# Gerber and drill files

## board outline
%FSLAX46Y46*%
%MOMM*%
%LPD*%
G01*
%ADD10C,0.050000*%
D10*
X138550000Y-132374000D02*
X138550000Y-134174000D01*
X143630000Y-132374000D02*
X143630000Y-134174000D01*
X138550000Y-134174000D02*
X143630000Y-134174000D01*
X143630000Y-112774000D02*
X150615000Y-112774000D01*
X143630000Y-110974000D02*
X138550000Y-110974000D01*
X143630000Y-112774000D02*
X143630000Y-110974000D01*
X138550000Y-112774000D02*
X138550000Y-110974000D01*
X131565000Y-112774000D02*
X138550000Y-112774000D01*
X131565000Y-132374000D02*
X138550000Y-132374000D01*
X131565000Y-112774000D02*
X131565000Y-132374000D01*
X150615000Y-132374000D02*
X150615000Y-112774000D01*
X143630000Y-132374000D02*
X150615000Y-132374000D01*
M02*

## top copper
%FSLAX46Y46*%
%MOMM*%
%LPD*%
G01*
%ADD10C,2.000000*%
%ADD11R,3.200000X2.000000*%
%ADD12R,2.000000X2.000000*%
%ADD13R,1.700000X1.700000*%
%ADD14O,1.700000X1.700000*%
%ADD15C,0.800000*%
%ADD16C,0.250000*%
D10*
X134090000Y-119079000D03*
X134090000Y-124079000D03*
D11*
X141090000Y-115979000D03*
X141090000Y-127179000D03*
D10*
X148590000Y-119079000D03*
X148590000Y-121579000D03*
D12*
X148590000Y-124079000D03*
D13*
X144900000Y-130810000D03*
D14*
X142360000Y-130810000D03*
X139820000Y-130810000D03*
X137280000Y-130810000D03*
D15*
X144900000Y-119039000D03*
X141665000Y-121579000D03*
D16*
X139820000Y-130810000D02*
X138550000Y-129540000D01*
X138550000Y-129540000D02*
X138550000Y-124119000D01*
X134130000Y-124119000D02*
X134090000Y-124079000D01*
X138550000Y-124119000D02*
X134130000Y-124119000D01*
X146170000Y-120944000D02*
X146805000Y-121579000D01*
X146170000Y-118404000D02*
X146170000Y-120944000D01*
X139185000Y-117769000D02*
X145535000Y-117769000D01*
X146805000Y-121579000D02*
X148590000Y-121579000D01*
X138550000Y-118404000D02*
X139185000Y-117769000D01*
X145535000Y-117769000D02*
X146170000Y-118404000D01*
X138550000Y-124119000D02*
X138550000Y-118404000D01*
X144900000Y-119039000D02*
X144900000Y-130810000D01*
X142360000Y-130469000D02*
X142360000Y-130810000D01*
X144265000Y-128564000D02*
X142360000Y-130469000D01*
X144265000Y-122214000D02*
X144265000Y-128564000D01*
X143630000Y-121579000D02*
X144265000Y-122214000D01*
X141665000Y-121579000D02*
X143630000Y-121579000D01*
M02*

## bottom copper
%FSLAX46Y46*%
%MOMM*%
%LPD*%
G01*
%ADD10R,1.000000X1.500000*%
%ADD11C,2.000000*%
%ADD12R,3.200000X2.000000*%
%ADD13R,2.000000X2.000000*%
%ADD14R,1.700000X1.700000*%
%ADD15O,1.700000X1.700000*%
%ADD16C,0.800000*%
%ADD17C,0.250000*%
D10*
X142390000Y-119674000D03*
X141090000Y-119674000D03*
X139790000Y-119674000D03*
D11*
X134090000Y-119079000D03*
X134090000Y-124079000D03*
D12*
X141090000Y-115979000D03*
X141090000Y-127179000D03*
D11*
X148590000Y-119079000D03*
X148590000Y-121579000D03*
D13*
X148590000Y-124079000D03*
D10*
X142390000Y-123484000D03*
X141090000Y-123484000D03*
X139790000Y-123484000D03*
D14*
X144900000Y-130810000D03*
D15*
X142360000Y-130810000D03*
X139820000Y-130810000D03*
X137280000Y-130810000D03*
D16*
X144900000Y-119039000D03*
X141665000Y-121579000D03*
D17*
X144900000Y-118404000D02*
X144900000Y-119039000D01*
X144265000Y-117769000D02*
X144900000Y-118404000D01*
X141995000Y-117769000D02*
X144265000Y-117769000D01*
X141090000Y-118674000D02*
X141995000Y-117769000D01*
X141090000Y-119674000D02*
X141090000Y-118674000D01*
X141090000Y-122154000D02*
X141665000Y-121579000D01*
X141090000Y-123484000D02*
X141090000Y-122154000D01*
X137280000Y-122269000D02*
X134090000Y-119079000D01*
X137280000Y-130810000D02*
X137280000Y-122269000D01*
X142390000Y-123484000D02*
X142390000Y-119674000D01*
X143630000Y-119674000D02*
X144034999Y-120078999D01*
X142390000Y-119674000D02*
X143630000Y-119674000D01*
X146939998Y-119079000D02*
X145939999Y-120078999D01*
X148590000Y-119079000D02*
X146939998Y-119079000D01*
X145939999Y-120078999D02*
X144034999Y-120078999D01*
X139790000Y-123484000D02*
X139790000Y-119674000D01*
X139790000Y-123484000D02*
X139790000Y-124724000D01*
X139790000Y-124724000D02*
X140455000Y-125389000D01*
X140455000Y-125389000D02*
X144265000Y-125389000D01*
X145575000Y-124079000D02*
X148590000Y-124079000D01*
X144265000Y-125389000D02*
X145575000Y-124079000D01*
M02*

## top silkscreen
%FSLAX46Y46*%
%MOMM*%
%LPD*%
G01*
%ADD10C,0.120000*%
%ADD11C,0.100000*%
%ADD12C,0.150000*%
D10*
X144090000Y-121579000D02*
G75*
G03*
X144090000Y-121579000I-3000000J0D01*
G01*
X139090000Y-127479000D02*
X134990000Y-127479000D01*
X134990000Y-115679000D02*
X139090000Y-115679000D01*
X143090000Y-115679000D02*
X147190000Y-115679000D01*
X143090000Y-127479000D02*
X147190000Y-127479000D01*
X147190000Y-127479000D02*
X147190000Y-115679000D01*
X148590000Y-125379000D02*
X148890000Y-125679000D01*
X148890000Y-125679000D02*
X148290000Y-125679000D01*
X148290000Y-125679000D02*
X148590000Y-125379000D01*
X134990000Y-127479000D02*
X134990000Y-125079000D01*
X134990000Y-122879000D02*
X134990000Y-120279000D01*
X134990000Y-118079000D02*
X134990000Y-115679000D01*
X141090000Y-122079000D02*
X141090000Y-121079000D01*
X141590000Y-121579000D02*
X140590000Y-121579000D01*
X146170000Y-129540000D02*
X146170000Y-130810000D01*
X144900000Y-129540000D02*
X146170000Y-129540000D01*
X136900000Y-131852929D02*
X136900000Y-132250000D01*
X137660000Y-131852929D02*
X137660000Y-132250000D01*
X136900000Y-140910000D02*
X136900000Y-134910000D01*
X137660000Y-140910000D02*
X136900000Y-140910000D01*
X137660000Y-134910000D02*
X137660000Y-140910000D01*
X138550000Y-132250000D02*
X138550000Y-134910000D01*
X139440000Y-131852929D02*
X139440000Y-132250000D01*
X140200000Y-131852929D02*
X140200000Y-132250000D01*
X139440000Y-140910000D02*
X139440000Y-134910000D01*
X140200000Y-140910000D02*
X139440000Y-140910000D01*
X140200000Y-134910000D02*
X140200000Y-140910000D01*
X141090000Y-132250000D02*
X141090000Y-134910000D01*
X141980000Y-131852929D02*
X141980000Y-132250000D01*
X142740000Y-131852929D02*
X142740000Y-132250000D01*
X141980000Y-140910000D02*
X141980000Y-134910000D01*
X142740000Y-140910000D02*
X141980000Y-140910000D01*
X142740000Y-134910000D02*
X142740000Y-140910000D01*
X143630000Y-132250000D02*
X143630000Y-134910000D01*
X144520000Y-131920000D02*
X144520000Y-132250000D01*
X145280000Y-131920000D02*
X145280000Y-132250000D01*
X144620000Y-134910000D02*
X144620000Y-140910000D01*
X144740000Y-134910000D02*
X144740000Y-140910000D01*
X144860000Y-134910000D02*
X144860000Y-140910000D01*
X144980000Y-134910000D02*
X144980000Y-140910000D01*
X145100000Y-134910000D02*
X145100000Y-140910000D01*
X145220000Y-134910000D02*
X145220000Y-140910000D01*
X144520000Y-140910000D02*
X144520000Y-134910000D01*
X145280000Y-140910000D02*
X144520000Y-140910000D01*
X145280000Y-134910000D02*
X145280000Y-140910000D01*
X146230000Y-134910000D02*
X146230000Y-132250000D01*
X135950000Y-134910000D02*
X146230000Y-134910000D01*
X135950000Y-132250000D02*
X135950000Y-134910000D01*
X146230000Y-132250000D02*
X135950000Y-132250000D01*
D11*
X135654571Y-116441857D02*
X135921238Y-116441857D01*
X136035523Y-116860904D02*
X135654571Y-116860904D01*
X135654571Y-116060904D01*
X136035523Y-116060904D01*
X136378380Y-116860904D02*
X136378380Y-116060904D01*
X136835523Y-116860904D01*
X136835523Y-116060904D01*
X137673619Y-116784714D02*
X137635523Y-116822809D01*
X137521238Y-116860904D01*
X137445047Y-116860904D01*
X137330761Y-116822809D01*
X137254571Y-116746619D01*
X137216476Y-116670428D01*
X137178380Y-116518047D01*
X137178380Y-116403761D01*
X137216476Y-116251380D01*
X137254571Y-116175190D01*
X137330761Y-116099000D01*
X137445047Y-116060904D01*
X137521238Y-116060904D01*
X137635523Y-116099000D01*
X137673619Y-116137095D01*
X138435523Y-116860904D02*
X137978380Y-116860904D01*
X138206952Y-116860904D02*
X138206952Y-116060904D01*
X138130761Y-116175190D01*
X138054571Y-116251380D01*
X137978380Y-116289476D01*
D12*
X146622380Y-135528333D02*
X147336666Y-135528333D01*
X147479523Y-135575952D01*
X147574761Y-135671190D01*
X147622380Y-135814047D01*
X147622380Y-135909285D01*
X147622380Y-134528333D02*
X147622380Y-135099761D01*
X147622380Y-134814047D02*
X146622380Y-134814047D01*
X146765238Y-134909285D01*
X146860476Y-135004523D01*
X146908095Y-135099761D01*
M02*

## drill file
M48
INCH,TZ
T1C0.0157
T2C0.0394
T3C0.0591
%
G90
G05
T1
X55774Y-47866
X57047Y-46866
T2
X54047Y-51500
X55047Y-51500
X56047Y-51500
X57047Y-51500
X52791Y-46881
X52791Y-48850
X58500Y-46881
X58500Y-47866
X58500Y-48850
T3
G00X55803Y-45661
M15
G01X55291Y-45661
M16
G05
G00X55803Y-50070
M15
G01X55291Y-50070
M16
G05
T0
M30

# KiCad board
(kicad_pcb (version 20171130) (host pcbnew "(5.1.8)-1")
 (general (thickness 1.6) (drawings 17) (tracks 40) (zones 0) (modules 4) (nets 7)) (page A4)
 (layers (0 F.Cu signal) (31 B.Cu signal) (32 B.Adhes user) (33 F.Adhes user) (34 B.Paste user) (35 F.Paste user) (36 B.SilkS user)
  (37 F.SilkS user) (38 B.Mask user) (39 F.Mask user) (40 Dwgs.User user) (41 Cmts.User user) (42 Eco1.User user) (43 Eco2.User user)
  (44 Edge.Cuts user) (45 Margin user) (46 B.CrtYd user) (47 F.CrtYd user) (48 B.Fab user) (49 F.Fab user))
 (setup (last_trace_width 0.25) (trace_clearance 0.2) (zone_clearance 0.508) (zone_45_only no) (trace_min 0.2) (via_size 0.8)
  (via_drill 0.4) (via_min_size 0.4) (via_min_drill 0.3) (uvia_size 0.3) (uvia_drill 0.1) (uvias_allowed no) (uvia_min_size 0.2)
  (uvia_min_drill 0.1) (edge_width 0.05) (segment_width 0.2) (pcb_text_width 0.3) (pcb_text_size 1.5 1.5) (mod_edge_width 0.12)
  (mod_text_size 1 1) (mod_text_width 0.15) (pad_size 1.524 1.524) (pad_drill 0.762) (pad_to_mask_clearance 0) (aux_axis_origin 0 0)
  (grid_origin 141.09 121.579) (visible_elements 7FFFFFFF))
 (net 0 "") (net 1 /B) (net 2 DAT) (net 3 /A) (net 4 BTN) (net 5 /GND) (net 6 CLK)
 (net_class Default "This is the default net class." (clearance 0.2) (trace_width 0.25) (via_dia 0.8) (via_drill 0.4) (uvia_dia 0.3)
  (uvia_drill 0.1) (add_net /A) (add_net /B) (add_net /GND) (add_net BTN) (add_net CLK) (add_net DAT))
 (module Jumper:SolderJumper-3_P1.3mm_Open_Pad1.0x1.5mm (layer B.Cu) (at 141.09 119.674 180)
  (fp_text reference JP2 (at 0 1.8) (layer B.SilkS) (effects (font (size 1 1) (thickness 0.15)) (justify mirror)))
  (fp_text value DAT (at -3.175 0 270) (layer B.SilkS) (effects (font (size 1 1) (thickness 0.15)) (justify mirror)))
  (pad 1 smd rect (at -1.3 0 180) (size 1 1.5) (layers B.Cu B.Mask) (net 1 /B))
  (pad 2 smd rect (at 0 0 180) (size 1 1.5) (layers B.Cu B.Mask) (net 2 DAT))
  (pad 3 smd rect (at 1.3 0 180) (size 1 1.5) (layers B.Cu B.Mask) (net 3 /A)))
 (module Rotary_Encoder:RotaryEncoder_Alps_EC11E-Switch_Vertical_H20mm (layer F.Cu) (at 148.59 124.079 180)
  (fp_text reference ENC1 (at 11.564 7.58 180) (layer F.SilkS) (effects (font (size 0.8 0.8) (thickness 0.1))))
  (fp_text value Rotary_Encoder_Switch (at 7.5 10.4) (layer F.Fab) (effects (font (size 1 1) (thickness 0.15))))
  (fp_circle (center 7.5 2.5) (end 10.5 2.5) (layer F.SilkS) (width 0.12))
  (fp_line (start 9.5 -3.4) (end 13.6 -3.4) (layer F.SilkS) (width 0.12))
  (fp_line (start 13.6 8.4) (end 9.5 8.4) (layer F.SilkS) (width 0.12))
  (fp_line (start 5.5 8.4) (end 1.4 8.4) (layer F.SilkS) (width 0.12))
  (fp_line (start 5.5 -3.4) (end 1.4 -3.4) (layer F.SilkS) (width 0.12))
  (fp_line (start 1.4 -3.4) (end 1.4 8.4) (layer F.SilkS) (width 0.12))
  (fp_line (start 0 -1.3) (end -0.3 -1.6) (layer F.SilkS) (width 0.12))
  (fp_line (start -0.3 -1.6) (end 0.3 -1.6) (layer F.SilkS) (width 0.12))
  (fp_line (start 0.3 -1.6) (end 0 -1.3) (layer F.SilkS) (width 0.12))
  (fp_line (start 13.6 -3.4) (end 13.6 -1) (layer F.SilkS) (width 0.12))
  (fp_line (start 13.6 1.2) (end 13.6 3.8) (layer F.SilkS) (width 0.12))
  (fp_line (start 13.6 6) (end 13.6 8.4) (layer F.SilkS) (width 0.12))
  (fp_line (start 7.5 2) (end 7.5 3) (layer F.SilkS) (width 0.12))
  (fp_line (start 7 2.5) (end 8 2.5) (layer F.SilkS) (width 0.12))
  (pad S1 thru_hole circle (at 14.5 5 180) (size 2 2) (drill 1) (layers *.Cu *.Mask) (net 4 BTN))
  (pad S2 thru_hole circle (at 14.5 0 180) (size 2 2) (drill 1) (layers *.Cu *.Mask) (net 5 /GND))
  (pad MP thru_hole rect (at 7.5 8.1 180) (size 3.2 2) (drill oval 2.8 1.5) (layers *.Cu *.Mask))
  (pad MP thru_hole rect (at 7.5 -3.1 180) (size 3.2 2) (drill oval 2.8 1.5) (layers *.Cu *.Mask))
  (pad B thru_hole circle (at 0 5 180) (size 2 2) (drill 1) (layers *.Cu *.Mask) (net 1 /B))
  (pad C thru_hole circle (at 0 2.5 180) (size 2 2) (drill 1) (layers *.Cu *.Mask) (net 5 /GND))
  (pad A thru_hole rect (at 0 0 180) (size 2 2) (drill 1) (layers *.Cu *.Mask) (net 3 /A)))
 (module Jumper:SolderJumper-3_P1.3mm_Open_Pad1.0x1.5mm (layer B.Cu) (at 141.09 123.484)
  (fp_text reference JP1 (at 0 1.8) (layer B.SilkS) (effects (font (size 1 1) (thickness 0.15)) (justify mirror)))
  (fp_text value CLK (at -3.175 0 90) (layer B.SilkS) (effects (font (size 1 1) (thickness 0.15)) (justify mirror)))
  (pad 3 smd rect (at 1.3 0) (size 1 1.5) (layers B.Cu B.Mask) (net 1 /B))
  (pad 2 smd rect (at 0 0) (size 1 1.5) (layers B.Cu B.Mask) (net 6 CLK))
  (pad 1 smd rect (at -1.3 0) (size 1 1.5) (layers B.Cu B.Mask) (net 3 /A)))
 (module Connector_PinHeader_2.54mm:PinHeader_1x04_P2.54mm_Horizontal (layer F.Cu) (at 144.9 130.81 270)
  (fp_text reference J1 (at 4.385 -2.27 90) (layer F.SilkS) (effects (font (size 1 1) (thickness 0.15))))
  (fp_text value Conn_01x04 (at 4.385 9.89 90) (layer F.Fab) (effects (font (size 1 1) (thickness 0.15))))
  (fp_line (start -1.27 -1.27) (end 0 -1.27) (layer F.SilkS) (width 0.12))
  (fp_line (start -1.27 0) (end -1.27 -1.27) (layer F.SilkS) (width 0.12))
  (fp_line (start 1.042929 8) (end 1.44 8) (layer F.SilkS) (width 0.12))
  (fp_line (start 1.042929 7.24) (end 1.44 7.24) (layer F.SilkS) (width 0.12))
  (fp_line (start 10.1 8) (end 4.1 8) (layer F.SilkS) (width 0.12))
  (fp_line (start 10.1 7.24) (end 10.1 8) (layer F.SilkS) (width 0.12))
  (fp_line (start 4.1 7.24) (end 10.1 7.24) (layer F.SilkS) (width 0.12))
  (fp_line (start 1.44 6.35) (end 4.1 6.35) (layer F.SilkS) (width 0.12))
  (fp_line (start 1.042929 5.46) (end 1.44 5.46) (layer F.SilkS) (width 0.12))
  (fp_line (start 1.042929 4.7) (end 1.44 4.7) (layer F.SilkS) (width 0.12))
  (fp_line (start 10.1 5.46) (end 4.1 5.46) (layer F.SilkS) (width 0.12))
  (fp_line (start 10.1 4.7) (end 10.1 5.46) (layer F.SilkS) (width 0.12))
  (fp_line (start 4.1 4.7) (end 10.1 4.7) (layer F.SilkS) (width 0.12))
  (fp_line (start 1.44 3.81) (end 4.1 3.81) (layer F.SilkS) (width 0.12))
  (fp_line (start 1.042929 2.92) (end 1.44 2.92) (layer F.SilkS) (width 0.12))
  (fp_line (start 1.042929 2.16) (end 1.44 2.16) (layer F.SilkS) (width 0.12))
  (fp_line (start 10.1 2.92) (end 4.1 2.92) (layer F.SilkS) (width 0.12))
  (fp_line (start 10.1 2.16) (end 10.1 2.92) (layer F.SilkS) (width 0.12))
  (fp_line (start 4.1 2.16) (end 10.1 2.16) (layer F.SilkS) (width 0.12))
  (fp_line (start 1.44 1.27) (end 4.1 1.27) (layer F.SilkS) (width 0.12))
  (fp_line (start 1.11 0.38) (end 1.44 0.38) (layer F.SilkS) (width 0.12))
  (fp_line (start 1.11 -0.38) (end 1.44 -0.38) (layer F.SilkS) (width 0.12))
  (fp_line (start 4.1 0.28) (end 10.1 0.28) (layer F.SilkS) (width 0.12))
  (fp_line (start 4.1 0.16) (end 10.1 0.16) (layer F.SilkS) (width 0.12))
  (fp_line (start 4.1 0.04) (end 10.1 0.04) (layer F.SilkS) (width 0.12))
  (fp_line (start 4.1 -0.08) (end 10.1 -0.08) (layer F.SilkS) (width 0.12))
  (fp_line (start 4.1 -0.2) (end 10.1 -0.2) (layer F.SilkS) (width 0.12))
  (fp_line (start 4.1 -0.32) (end 10.1 -0.32) (layer F.SilkS) (width 0.12))
  (fp_line (start 10.1 0.38) (end 4.1 0.38) (layer F.SilkS) (width 0.12))
  (fp_line (start 10.1 -0.38) (end 10.1 0.38) (layer F.SilkS) (width 0.12))
  (fp_line (start 4.1 -0.38) (end 10.1 -0.38) (layer F.SilkS) (width 0.12))
  (fp_line (start 4.1 -1.33) (end 1.44 -1.33) (layer F.SilkS) (width 0.12))
  (fp_line (start 4.1 8.95) (end 4.1 -1.33) (layer F.SilkS) (width 0.12))
  (fp_line (start 1.44 8.95) (end 4.1 8.95) (layer F.SilkS) (width 0.12))
  (fp_line (start 1.44 -1.33) (end 1.44 8.95) (layer F.SilkS) (width 0.12))
  (pad 1 thru_hole rect (at 0 0 270) (size 1.7 1.7) (drill 1) (layers *.Cu *.Mask) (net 2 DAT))
  (pad 2 thru_hole oval (at 0 2.54 270) (size 1.7 1.7) (drill 1) (layers *.Cu *.Mask) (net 6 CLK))
  (pad 3 thru_hole oval (at 0 5.08 270) (size 1.7 1.7) (drill 1) (layers *.Cu *.Mask) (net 5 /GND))
  (pad 4 thru_hole oval (at 0 7.62 270) (size 1.7 1.7) (drill 1) (layers *.Cu *.Mask) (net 4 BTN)))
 (gr_line (start 138.55 132.374) (end 138.55 134.174) (layer Edge.Cuts) (width 0.05))
 (gr_line (start 143.63 132.374) (end 143.63 134.174) (layer Edge.Cuts) (width 0.05))
 (gr_line (start 138.55 134.174) (end 143.63 134.174) (layer Edge.Cuts) (width 0.05))
 (gr_line (start 143.63 112.774) (end 150.615 112.774) (layer Edge.Cuts) (width 0.05))
 (gr_line (start 143.63 110.974) (end 138.55 110.974) (layer Edge.Cuts) (width 0.05))
 (gr_line (start 143.63 112.774) (end 143.63 110.974) (layer Edge.Cuts) (width 0.05))
 (gr_line (start 138.55 112.774) (end 138.55 110.974) (layer Edge.Cuts) (width 0.05))
 (gr_line (start 131.565 112.774) (end 138.55 112.774) (layer Edge.Cuts) (width 0.05))
 (gr_line (start 131.565 132.374) (end 138.55 132.374) (layer Edge.Cuts) (width 0.05))
 (gr_line (start 131.565 112.774) (end 131.565 132.374) (layer Edge.Cuts) (width 0.05))
 (gr_line (start 150.615 132.374) (end 150.615 112.774) (layer Edge.Cuts) (width 0.05))
 (gr_line (start 143.63 132.374) (end 150.615 132.374) (layer Edge.Cuts) (width 0.05))
 (segment (start 139.82 130.81) (end 138.55 129.54) (width 0.25) (layer F.Cu) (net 5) (status 10))
 (segment (start 138.55 129.54) (end 138.55 124.119) (width 0.25) (layer F.Cu) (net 5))
 (segment (start 134.13 124.119) (end 134.09 124.079) (width 0.25) (layer F.Cu) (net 5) (status 30))
 (segment (start 138.55 124.119) (end 134.13 124.119) (width 0.25) (layer F.Cu) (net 5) (status 20))
 (segment (start 146.17 120.944) (end 146.805 121.579) (width 0.25) (layer F.Cu) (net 5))
 (segment (start 146.17 118.404) (end 146.17 120.944) (width 0.25) (layer F.Cu) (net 5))
 (segment (start 139.185 117.769) (end 145.535 117.769) (width 0.25) (layer F.Cu) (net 5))
 (segment (start 146.805 121.579) (end 148.59 121.579) (width 0.25) (layer F.Cu) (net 5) (status 20))
 (segment (start 138.55 118.404) (end 139.185 117.769) (width 0.25) (layer F.Cu) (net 5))
 (segment (start 145.535 117.769) (end 146.17 118.404) (width 0.25) (layer F.Cu) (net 5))
 (segment (start 138.55 124.119) (end 138.55 118.404) (width 0.25) (layer F.Cu) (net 5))
 (via (at 144.9 119.039) (size 0.8) (drill 0.4) (layers F.Cu B.Cu) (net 2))
 (segment (start 144.9 118.404) (end 144.9 119.039) (width 0.25) (layer B.Cu) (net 2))
 (segment (start 144.265 117.769) (end 144.9 118.404) (width 0.25) (layer B.Cu) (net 2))
 (segment (start 141.995 117.769) (end 144.265 117.769) (width 0.25) (layer B.Cu) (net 2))
 (segment (start 141.09 118.674) (end 141.995 117.769) (width 0.25) (layer B.Cu) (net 2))
 (segment (start 141.09 119.674) (end 141.09 118.674) (width 0.25) (layer B.Cu) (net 2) (status 10))
 (segment (start 144.9 119.039) (end 144.9 130.81) (width 0.25) (layer F.Cu) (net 2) (status 20))
 (via (at 141.665 121.579) (size 0.8) (drill 0.4) (layers F.Cu B.Cu) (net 6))
 (segment (start 141.09 122.154) (end 141.665 121.579) (width 0.25) (layer B.Cu) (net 6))
 (segment (start 141.09 123.484) (end 141.09 122.154) (width 0.25) (layer B.Cu) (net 6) (status 10))
 (segment (start 142.36 130.469) (end 142.36 130.81) (width 0.25) (layer F.Cu) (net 6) (status 30))
 (segment (start 144.265 128.564) (end 142.36 130.469) (width 0.25) (layer F.Cu) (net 6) (status 20))
 (segment (start 144.265 122.214) (end 144.265 128.564) (width 0.25) (layer F.Cu) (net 6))
 (segment (start 143.63 121.579) (end 144.265 122.214) (width 0.25) (layer F.Cu) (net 6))
 (segment (start 141.665 121.579) (end 143.63 121.579) (width 0.25) (layer F.Cu) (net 6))
 (segment (start 137.28 122.269) (end 134.09 119.079) (width 0.25) (layer B.Cu) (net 4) (status 20))
 (segment (start 137.28 130.81) (end 137.28 122.269) (width 0.25) (layer B.Cu) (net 4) (status 10))
 (segment (start 142.39 123.484) (end 142.39 119.674) (width 0.25) (layer B.Cu) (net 1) (status 30))
 (segment (start 143.63 119.674) (end 144.034999 120.078999) (width 0.25) (layer B.Cu) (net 1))
 (segment (start 142.39 119.674) (end 143.63 119.674) (width 0.25) (layer B.Cu) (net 1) (status 10))
 (segment (start 146.939998 119.079) (end 145.939999 120.078999) (width 0.25) (layer B.Cu) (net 1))
 (segment (start 148.59 119.079) (end 146.939998 119.079) (width 0.25) (layer B.Cu) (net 1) (status 10))
 (segment (start 145.939999 120.078999) (end 144.034999 120.078999) (width 0.25) (layer B.Cu) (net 1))
 (segment (start 139.79 123.484) (end 139.79 119.674) (width 0.25) (layer B.Cu) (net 3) (status 30))
 (segment (start 139.79 123.484) (end 139.79 124.724) (width 0.25) (layer B.Cu) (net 3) (status 10))
 (segment (start 139.79 124.724) (end 140.455 125.389) (width 0.25) (layer B.Cu) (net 3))
 (segment (start 140.455 125.389) (end 144.265 125.389) (width 0.25) (layer B.Cu) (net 3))
 (segment (start 145.575 124.079) (end 148.59 124.079) (width 0.25) (layer B.Cu) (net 3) (status 20))
 (segment (start 144.265 125.389) (end 145.575 124.079) (width 0.25) (layer B.Cu) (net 3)))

